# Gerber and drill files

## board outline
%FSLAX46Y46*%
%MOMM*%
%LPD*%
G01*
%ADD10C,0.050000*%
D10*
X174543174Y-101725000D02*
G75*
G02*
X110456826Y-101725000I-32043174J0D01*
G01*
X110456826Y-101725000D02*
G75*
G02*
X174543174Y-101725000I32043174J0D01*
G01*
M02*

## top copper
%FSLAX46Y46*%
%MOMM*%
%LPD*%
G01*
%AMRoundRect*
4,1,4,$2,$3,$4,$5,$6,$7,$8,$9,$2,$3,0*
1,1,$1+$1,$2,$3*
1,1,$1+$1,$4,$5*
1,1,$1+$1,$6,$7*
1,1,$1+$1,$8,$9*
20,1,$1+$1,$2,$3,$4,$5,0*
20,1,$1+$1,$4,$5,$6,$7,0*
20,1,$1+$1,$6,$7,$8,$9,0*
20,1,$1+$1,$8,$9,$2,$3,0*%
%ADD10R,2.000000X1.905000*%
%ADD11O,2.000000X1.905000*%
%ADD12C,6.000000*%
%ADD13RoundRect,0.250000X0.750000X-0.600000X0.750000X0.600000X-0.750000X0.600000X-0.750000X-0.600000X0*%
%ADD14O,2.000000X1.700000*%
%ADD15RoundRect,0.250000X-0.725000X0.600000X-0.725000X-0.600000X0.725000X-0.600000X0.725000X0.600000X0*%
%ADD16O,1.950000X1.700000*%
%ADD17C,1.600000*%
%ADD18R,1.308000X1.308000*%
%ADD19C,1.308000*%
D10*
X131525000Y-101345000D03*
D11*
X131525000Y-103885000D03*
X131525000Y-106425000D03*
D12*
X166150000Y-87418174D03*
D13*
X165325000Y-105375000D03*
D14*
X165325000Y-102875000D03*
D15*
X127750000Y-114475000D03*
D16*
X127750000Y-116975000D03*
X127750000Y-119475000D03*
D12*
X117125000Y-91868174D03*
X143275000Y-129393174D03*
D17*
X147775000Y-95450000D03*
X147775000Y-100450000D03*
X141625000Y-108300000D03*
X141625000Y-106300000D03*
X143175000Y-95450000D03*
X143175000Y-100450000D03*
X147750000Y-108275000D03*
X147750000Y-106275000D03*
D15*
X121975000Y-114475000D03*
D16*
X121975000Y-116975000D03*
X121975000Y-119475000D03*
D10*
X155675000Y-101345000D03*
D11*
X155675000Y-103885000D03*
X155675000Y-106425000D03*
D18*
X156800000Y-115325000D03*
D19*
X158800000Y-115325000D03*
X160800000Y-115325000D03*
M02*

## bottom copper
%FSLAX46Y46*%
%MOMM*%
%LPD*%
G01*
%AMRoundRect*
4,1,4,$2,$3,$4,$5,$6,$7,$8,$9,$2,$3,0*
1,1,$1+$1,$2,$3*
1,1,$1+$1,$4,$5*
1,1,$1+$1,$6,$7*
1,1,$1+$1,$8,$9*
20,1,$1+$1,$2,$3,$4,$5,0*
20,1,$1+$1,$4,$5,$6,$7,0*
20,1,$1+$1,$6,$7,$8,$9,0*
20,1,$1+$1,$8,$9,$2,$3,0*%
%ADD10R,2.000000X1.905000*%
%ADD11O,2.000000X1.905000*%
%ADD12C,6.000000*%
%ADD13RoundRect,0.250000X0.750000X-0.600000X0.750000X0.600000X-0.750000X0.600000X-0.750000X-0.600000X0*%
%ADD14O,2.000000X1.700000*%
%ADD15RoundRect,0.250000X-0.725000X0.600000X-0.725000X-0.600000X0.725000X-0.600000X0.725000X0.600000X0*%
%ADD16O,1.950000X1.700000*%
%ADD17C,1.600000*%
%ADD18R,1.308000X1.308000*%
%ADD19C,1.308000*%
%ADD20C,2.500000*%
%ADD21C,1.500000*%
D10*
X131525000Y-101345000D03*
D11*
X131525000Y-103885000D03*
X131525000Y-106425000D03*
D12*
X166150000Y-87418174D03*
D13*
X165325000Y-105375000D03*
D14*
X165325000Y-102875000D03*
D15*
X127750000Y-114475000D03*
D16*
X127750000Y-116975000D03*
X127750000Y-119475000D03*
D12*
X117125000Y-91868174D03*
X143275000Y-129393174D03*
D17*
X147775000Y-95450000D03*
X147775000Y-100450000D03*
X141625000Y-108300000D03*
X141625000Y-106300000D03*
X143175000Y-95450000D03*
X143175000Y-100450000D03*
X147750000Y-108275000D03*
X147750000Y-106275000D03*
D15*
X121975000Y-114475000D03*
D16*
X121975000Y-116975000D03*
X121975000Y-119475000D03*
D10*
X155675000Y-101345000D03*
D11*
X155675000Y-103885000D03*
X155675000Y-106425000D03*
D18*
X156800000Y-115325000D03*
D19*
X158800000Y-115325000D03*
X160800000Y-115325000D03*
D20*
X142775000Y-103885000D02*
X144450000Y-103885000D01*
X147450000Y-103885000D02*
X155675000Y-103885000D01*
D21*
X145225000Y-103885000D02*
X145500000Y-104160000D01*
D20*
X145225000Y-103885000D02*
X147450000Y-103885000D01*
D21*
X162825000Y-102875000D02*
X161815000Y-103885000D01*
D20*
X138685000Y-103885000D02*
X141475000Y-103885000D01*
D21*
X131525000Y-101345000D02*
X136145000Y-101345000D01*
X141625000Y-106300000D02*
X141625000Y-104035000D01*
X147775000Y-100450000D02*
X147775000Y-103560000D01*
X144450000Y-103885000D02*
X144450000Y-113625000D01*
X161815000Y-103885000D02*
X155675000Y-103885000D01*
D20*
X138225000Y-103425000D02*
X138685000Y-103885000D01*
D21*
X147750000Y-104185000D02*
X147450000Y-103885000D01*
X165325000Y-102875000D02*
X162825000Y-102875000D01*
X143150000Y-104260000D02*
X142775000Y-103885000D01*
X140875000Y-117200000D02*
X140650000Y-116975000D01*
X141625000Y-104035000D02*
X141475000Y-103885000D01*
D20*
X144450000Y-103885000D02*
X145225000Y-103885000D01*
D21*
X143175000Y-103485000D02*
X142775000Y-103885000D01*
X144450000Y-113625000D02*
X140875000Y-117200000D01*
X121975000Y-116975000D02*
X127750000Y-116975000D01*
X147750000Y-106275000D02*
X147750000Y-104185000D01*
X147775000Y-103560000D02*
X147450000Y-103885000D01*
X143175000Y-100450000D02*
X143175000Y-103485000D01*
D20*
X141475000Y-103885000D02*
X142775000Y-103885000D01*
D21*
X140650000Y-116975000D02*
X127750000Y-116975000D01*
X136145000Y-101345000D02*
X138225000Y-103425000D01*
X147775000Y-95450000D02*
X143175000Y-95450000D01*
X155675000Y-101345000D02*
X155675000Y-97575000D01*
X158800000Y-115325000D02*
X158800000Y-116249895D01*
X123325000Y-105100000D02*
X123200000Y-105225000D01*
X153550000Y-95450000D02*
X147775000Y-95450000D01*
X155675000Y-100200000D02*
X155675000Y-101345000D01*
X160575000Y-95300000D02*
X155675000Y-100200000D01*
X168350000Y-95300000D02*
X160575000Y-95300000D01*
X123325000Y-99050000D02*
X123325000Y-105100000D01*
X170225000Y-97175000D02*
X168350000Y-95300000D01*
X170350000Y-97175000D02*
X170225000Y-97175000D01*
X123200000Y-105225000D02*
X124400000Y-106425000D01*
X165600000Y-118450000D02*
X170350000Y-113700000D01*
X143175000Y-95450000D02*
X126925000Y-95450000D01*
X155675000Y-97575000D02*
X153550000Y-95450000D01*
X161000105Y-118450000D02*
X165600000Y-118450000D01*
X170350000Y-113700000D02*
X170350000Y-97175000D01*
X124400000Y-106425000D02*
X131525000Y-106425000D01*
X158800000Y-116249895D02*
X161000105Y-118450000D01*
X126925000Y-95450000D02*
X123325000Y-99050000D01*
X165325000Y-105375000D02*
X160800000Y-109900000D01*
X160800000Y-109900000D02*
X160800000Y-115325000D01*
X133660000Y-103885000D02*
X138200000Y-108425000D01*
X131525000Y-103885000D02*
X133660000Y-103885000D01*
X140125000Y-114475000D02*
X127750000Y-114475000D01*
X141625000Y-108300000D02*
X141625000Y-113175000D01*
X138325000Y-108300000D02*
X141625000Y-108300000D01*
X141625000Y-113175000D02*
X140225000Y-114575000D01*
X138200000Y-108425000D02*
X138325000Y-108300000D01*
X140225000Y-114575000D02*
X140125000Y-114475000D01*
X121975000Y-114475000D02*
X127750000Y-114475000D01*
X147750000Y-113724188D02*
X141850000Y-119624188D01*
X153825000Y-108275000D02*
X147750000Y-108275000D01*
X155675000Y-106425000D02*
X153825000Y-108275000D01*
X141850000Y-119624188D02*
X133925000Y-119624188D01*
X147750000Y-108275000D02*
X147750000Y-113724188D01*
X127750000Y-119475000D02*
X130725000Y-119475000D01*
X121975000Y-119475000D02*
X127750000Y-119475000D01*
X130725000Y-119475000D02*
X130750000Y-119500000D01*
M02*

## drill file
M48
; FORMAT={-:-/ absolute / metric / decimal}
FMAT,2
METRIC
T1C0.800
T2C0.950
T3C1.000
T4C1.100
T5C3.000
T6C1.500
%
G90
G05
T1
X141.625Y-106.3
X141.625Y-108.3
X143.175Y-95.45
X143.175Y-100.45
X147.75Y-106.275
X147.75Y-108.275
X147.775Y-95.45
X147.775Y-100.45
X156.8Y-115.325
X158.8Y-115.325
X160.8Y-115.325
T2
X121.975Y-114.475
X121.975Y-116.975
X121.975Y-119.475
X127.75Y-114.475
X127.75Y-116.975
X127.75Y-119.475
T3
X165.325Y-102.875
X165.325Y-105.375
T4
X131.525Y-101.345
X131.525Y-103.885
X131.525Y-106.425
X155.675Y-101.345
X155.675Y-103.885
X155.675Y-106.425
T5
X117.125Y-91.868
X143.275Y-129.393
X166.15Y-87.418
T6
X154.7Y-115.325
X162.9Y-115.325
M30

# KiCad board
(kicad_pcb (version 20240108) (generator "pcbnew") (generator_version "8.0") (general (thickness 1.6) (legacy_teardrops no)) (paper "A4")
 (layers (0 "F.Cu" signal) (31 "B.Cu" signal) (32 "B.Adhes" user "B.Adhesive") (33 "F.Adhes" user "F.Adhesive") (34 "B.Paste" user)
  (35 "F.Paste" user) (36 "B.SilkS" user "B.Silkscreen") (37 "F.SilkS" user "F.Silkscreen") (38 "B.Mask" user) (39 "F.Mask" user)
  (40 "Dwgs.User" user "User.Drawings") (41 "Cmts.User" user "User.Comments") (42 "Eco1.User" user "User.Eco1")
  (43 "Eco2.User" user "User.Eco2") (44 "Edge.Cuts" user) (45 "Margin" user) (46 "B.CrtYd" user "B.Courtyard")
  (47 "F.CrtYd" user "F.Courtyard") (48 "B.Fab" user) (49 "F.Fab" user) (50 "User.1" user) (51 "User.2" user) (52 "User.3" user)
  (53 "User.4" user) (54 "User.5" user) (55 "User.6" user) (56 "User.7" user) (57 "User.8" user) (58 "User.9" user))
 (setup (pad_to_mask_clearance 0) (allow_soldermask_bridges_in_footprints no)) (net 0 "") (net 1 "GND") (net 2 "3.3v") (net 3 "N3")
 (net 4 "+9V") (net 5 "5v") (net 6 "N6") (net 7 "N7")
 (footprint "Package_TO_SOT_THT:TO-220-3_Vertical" (layer "F.Cu") (at 131.525 101.345 -90)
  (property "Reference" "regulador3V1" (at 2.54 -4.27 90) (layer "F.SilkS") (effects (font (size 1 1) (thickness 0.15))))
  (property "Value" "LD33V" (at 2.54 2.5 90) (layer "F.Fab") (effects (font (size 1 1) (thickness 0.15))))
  (pad "1" thru_hole rect (at 0 0 270) (size 1.905 2) (drill 1.1) (layers "*.Cu" "*.Mask") (remove_unused_layers no) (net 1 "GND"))
  (pad "2" thru_hole oval (at 2.54 0 270) (size 1.905 2) (drill 1.1) (layers "*.Cu" "*.Mask") (remove_unused_layers no) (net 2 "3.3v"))
  (pad "3" thru_hole oval (at 5.08 0 270) (size 1.905 2) (drill 1.1) (layers "*.Cu" "*.Mask") (remove_unused_layers no) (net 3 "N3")))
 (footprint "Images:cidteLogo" (layer "F.Cu") (at 142.25 102.318174 180)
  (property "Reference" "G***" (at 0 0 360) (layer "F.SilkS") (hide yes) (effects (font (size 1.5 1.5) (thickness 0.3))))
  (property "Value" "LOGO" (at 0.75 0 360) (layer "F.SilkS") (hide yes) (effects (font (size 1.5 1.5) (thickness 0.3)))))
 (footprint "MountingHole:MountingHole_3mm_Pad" (layer "F.Cu") (at 166.15 87.418174)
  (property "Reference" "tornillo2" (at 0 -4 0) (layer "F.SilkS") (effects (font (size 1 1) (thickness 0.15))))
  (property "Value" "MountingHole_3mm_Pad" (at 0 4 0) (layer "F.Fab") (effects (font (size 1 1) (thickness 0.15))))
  (pad "2" thru_hole circle (at 0 0) (size 6 6) (drill 3) (layers "*.Cu" "*.Mask") (remove_unused_layers no)))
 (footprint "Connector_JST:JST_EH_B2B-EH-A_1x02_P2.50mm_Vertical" (layer "F.Cu") (at 165.325 105.375 90)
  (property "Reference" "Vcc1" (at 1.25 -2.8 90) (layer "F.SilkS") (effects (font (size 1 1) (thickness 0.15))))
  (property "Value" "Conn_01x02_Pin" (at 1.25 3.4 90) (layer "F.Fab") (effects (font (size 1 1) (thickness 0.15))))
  (pad "1" thru_hole roundrect (at 0 0 90) (size 1.7 2) (drill 1) (layers "*.Cu" "*.Mask") (remove_unused_layers no)
   (roundrect_rratio 0.147059) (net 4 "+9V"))
  (pad "2" thru_hole oval (at 2.5 0 90) (size 1.7 2) (drill 1) (layers "*.Cu" "*.Mask") (remove_unused_layers no) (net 1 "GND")))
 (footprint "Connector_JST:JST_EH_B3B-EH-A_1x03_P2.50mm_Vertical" (layer "F.Cu") (at 127.75 114.475 -90)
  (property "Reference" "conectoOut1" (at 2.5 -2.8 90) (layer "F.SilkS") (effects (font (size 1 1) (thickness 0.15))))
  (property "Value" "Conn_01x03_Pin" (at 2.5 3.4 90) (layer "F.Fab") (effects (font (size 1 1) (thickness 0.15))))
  (pad "1" thru_hole roundrect (at 0 0 270) (size 1.7 1.95) (drill 0.95) (layers "*.Cu" "*.Mask") (remove_unused_layers no)
   (roundrect_rratio 0.147059) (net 2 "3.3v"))
  (pad "2" thru_hole oval (at 2.5 0 270) (size 1.7 1.95) (drill 0.95) (layers "*.Cu" "*.Mask") (remove_unused_layers no) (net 1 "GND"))
  (pad "3" thru_hole oval (at 5 0 270) (size 1.7 1.95) (drill 0.95) (layers "*.Cu" "*.Mask") (remove_unused_layers no) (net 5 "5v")))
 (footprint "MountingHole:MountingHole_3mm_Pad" (layer "F.Cu") (at 117.125 91.868174)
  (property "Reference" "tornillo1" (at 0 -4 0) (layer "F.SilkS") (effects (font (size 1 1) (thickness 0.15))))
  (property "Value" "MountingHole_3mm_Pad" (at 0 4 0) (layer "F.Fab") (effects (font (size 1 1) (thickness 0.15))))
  (pad "1" thru_hole circle (at 0 0) (size 6 6) (drill 3) (layers "*.Cu" "*.Mask") (remove_unused_layers no)))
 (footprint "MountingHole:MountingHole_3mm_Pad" (layer "F.Cu") (at 143.275 129.393174)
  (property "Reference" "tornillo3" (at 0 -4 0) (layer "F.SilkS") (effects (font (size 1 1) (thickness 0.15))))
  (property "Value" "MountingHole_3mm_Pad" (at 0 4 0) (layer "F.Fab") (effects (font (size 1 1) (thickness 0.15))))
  (pad "3" thru_hole circle (at 0 0) (size 6 6) (drill 3) (layers "*.Cu" "*.Mask") (remove_unused_layers no)))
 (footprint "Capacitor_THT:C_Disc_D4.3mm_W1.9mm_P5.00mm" (layer "F.Cu") (at 147.775 95.45 -90)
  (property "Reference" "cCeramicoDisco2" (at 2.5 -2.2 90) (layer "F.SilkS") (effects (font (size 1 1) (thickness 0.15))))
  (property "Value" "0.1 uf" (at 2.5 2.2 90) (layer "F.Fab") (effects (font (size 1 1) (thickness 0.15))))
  (pad "1" thru_hole circle (at 0 0 270) (size 1.6 1.6) (drill 0.8) (layers "*.Cu" "*.Mask") (remove_unused_layers no) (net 3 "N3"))
  (pad "2" thru_hole circle (at 5 0 270) (size 1.6 1.6) (drill 0.8) (layers "*.Cu" "*.Mask") (remove_unused_layers no) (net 1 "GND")))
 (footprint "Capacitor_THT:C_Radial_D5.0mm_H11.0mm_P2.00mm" (layer "F.Cu") (at 141.625 108.3 90)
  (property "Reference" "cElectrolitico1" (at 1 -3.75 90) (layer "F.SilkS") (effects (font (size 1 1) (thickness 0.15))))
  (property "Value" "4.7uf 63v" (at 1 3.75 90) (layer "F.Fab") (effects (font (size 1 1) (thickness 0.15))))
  (pad "1" thru_hole circle (at 0 0 90) (size 1.6 1.6) (drill 0.8) (layers "*.Cu" "*.Mask") (remove_unused_layers no) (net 2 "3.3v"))
  (pad "2" thru_hole circle (at 2 0 90) (size 1.6 1.6) (drill 0.8) (layers "*.Cu" "*.Mask") (remove_unused_layers no) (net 1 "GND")))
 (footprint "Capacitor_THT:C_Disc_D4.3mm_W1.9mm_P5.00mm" (layer "F.Cu") (at 143.175 95.45 -90)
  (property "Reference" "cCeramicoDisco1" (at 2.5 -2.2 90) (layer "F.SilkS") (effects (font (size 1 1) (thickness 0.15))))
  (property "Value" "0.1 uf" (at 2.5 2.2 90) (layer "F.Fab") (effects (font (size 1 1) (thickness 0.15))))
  (pad "1" thru_hole circle (at 0 0 270) (size 1.6 1.6) (drill 0.8) (layers "*.Cu" "*.Mask") (remove_unused_layers no) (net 3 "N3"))
  (pad "2" thru_hole circle (at 5 0 270) (size 1.6 1.6) (drill 0.8) (layers "*.Cu" "*.Mask") (remove_unused_layers no) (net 1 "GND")))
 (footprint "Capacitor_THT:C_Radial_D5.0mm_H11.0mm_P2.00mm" (layer "F.Cu") (at 147.75 108.275 90)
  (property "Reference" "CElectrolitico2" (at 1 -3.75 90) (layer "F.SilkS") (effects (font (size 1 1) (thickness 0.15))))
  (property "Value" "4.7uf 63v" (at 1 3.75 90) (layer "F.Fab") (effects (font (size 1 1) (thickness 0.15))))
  (pad "1" thru_hole circle (at 0 0 90) (size 1.6 1.6) (drill 0.8) (layers "*.Cu" "*.Mask") (remove_unused_layers no) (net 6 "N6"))
  (pad "2" thru_hole circle (at 2 0 90) (size 1.6 1.6) (drill 0.8) (layers "*.Cu" "*.Mask") (remove_unused_layers no) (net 1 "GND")))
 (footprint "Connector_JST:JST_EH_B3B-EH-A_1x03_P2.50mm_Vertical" (layer "F.Cu") (at 121.975 114.475 -90)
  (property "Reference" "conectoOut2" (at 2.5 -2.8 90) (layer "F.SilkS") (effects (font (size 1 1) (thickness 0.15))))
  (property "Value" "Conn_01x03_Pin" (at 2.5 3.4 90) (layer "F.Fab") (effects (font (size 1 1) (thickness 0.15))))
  (pad "1" thru_hole roundrect (at 0 0 270) (size 1.7 1.95) (drill 0.95) (layers "*.Cu" "*.Mask") (remove_unused_layers no)
   (roundrect_rratio 0.147059) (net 2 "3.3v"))
  (pad "2" thru_hole oval (at 2.5 0 270) (size 1.7 1.95) (drill 0.95) (layers "*.Cu" "*.Mask") (remove_unused_layers no) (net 1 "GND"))
  (pad "3" thru_hole oval (at 5 0 270) (size 1.7 1.95) (drill 0.95) (layers "*.Cu" "*.Mask") (remove_unused_layers no) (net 5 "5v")))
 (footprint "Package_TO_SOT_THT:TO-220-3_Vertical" (layer "F.Cu") (at 155.675 101.345 -90)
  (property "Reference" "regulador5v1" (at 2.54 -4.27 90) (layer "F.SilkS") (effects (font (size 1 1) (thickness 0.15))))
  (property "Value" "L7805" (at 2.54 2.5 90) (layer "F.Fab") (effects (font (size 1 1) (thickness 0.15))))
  (pad "1" thru_hole rect (at 0 0 270) (size 1.905 2) (drill 1.1) (layers "*.Cu" "*.Mask") (remove_unused_layers no) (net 3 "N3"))
  (pad "2" thru_hole oval (at 2.54 0 270) (size 1.905 2) (drill 1.1) (layers "*.Cu" "*.Mask") (remove_unused_layers no) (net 1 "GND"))
  (pad "3" thru_hole oval (at 5.08 0 270) (size 1.905 2) (drill 1.1) (layers "*.Cu" "*.Mask") (remove_unused_layers no) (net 6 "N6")))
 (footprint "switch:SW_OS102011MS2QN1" (layer "F.Cu") (at 158.8 115.325)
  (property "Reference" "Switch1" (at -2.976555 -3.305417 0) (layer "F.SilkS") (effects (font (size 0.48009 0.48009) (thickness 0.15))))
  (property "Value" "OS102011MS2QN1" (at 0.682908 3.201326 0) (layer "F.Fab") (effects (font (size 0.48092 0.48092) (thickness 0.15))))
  (pad "" np_thru_hole circle (at -4.1 0) (size 1.5 1.5) (drill 1.5) (layers "*.Cu" "*.Mask"))
  (pad "" np_thru_hole circle (at 4.1 0) (size 1.5 1.5) (drill 1.5) (layers "*.Cu" "*.Mask"))
  (pad "1" thru_hole rect (at -2 0) (size 1.308 1.308) (drill 0.8) (layers "*.Cu" "*.Mask") (remove_unused_layers no) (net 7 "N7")
   (solder_mask_margin 0.102))
  (pad "2" thru_hole circle (at 0 0) (size 1.308 1.308) (drill 0.8) (layers "*.Cu" "*.Mask") (remove_unused_layers no) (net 3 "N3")
   (solder_mask_margin 0.102))
  (pad "3" thru_hole circle (at 2 0) (size 1.308 1.308) (drill 0.8) (layers "*.Cu" "*.Mask") (remove_unused_layers no) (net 4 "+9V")
   (solder_mask_margin 0.102)))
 (gr_circle (center 142.5 101.725) (end 164.55 124.975) (stroke (width 0.05) (type default)) (fill none) (layer "Edge.Cuts"))
 (segment (start 142.775 103.885) (end 144.45 103.885) (width 2.5) (layer "B.Cu") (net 1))
 (segment (start 147.45 103.885) (end 155.675 103.885) (width 2.5) (layer "B.Cu") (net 1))
 (segment (start 145.225 103.885) (end 145.5 104.16) (width 1.5) (layer "B.Cu") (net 1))
 (segment (start 145.225 103.885) (end 147.45 103.885) (width 2.5) (layer "B.Cu") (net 1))
 (segment (start 162.825 102.875) (end 161.815 103.885) (width 1.5) (layer "B.Cu") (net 1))
 (segment (start 138.685 103.885) (end 141.475 103.885) (width 2.5) (layer "B.Cu") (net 1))
 (segment (start 131.525 101.345) (end 136.145 101.345) (width 1.5) (layer "B.Cu") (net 1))
 (segment (start 141.625 106.3) (end 141.625 104.035) (width 1.5) (layer "B.Cu") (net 1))
 (segment (start 147.775 100.45) (end 147.775 103.56) (width 1.5) (layer "B.Cu") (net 1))
 (segment (start 144.45 103.885) (end 144.45 113.625) (width 1.5) (layer "B.Cu") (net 1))
 (segment (start 161.815 103.885) (end 155.675 103.885) (width 1.5) (layer "B.Cu") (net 1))
 (segment (start 138.225 103.425) (end 138.685 103.885) (width 2.5) (layer "B.Cu") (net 1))
 (segment (start 147.75 104.185) (end 147.45 103.885) (width 1.5) (layer "B.Cu") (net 1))
 (segment (start 165.325 102.875) (end 162.825 102.875) (width 1.5) (layer "B.Cu") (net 1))
 (segment (start 143.15 104.26) (end 142.775 103.885) (width 1.5) (layer "B.Cu") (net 1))
 (segment (start 140.875 117.2) (end 140.65 116.975) (width 1.5) (layer "B.Cu") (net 1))
 (segment (start 141.625 104.035) (end 141.475 103.885) (width 1.5) (layer "B.Cu") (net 1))
 (segment (start 144.45 103.885) (end 145.225 103.885) (width 2.5) (layer "B.Cu") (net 1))
 (segment (start 143.175 103.485) (end 142.775 103.885) (width 1.5) (layer "B.Cu") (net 1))
 (segment (start 144.45 113.625) (end 140.875 117.2) (width 1.5) (layer "B.Cu") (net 1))
 (segment (start 121.975 116.975) (end 127.75 116.975) (width 1.5) (layer "B.Cu") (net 1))
 (segment (start 147.75 106.275) (end 147.75 104.185) (width 1.5) (layer "B.Cu") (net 1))
 (segment (start 147.775 103.56) (end 147.45 103.885) (width 1.5) (layer "B.Cu") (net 1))
 (segment (start 143.175 100.45) (end 143.175 103.485) (width 1.5) (layer "B.Cu") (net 1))
 (segment (start 141.475 103.885) (end 142.775 103.885) (width 2.5) (layer "B.Cu") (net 1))
 (segment (start 140.65 116.975) (end 127.75 116.975) (width 1.5) (layer "B.Cu") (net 1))
 (segment (start 136.145 101.345) (end 138.225 103.425) (width 1.5) (layer "B.Cu") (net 1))
 (segment (start 147.775 95.45) (end 143.175 95.45) (width 1.5) (layer "B.Cu") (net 3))
 (segment (start 155.675 101.345) (end 155.675 97.575) (width 1.5) (layer "B.Cu") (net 3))
 (segment (start 158.8 115.325) (end 158.8 116.249895) (width 1.5) (layer "B.Cu") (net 3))
 (segment (start 123.325 105.1) (end 123.2 105.225) (width 1.5) (layer "B.Cu") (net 3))
 (segment (start 153.55 95.45) (end 147.775 95.45) (width 1.5) (layer "B.Cu") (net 3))
 (segment (start 155.675 100.2) (end 155.675 101.345) (width 1.5) (layer "B.Cu") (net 3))
 (segment (start 160.575 95.3) (end 155.675 100.2) (width 1.5) (layer "B.Cu") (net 3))
 (segment (start 168.35 95.3) (end 160.575 95.3) (width 1.5) (layer "B.Cu") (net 3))
 (segment (start 123.325 99.05) (end 123.325 105.1) (width 1.5) (layer "B.Cu") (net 3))
 (segment (start 170.225 97.175) (end 168.35 95.3) (width 1.5) (layer "B.Cu") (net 3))
 (segment (start 170.35 97.175) (end 170.225 97.175) (width 1.5) (layer "B.Cu") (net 3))
 (segment (start 123.2 105.225) (end 124.4 106.425) (width 1.5) (layer "B.Cu") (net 3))
 (segment (start 165.6 118.45) (end 170.35 113.7) (width 1.5) (layer "B.Cu") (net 3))
 (segment (start 143.175 95.45) (end 126.925 95.45) (width 1.5) (layer "B.Cu") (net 3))
 (segment (start 155.675 97.575) (end 153.55 95.45) (width 1.5) (layer "B.Cu") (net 3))
 (segment (start 161.000105 118.45) (end 165.6 118.45) (width 1.5) (layer "B.Cu") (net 3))
 (segment (start 170.35 113.7) (end 170.35 97.175) (width 1.5) (layer "B.Cu") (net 3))
 (segment (start 124.4 106.425) (end 131.525 106.425) (width 1.5) (layer "B.Cu") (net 3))
 (segment (start 158.8 116.249895) (end 161.000105 118.45) (width 1.5) (layer "B.Cu") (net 3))
 (segment (start 126.925 95.45) (end 123.325 99.05) (width 1.5) (layer "B.Cu") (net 3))
 (segment (start 165.325 105.375) (end 160.8 109.9) (width 1.5) (layer "B.Cu") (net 4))
 (segment (start 160.8 109.9) (end 160.8 115.325) (width 1.5) (layer "B.Cu") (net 4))
 (segment (start 133.66 103.885) (end 138.2 108.425) (width 1.5) (layer "B.Cu") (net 2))
 (segment (start 131.525 103.885) (end 133.66 103.885) (width 1.5) (layer "B.Cu") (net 2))
 (segment (start 140.125 114.475) (end 127.75 114.475) (width 1.5) (layer "B.Cu") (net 2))
 (segment (start 141.625 108.3) (end 141.625 113.175) (width 1.5) (layer "B.Cu") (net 2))
 (segment (start 138.325 108.3) (end 141.625 108.3) (width 1.5) (layer "B.Cu") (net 2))
 (segment (start 141.625 113.175) (end 140.225 114.575) (width 1.5) (layer "B.Cu") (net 2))
 (segment (start 138.2 108.425) (end 138.325 108.3) (width 1.5) (layer "B.Cu") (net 2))
 (segment (start 140.225 114.575) (end 140.125 114.475) (width 1.5) (layer "B.Cu") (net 2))
 (segment (start 121.975 114.475) (end 127.75 114.475) (width 1.5) (layer "B.Cu") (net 2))
 (segment (start 147.75 113.724188) (end 141.85 119.624188) (width 1.5) (layer "B.Cu") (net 6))
 (segment (start 153.825 108.275) (end 147.75 108.275) (width 1.5) (layer "B.Cu") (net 6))
 (segment (start 155.675 106.425) (end 153.825 108.275) (width 1.5) (layer "B.Cu") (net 6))
 (segment (start 141.85 119.624188) (end 133.925 119.624188) (width 1.5) (layer "B.Cu") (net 6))
 (segment (start 147.75 108.275) (end 147.75 113.724188) (width 1.5) (layer "B.Cu") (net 6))
 (segment (start 127.75 119.475) (end 130.725 119.475) (width 1.5) (layer "B.Cu") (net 5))
 (segment (start 121.975 119.475) (end 127.75 119.475) (width 1.5) (layer "B.Cu") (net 5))
 (segment (start 130.725 119.475) (end 130.75 119.5) (width 1.5) (layer "B.Cu") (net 5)))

